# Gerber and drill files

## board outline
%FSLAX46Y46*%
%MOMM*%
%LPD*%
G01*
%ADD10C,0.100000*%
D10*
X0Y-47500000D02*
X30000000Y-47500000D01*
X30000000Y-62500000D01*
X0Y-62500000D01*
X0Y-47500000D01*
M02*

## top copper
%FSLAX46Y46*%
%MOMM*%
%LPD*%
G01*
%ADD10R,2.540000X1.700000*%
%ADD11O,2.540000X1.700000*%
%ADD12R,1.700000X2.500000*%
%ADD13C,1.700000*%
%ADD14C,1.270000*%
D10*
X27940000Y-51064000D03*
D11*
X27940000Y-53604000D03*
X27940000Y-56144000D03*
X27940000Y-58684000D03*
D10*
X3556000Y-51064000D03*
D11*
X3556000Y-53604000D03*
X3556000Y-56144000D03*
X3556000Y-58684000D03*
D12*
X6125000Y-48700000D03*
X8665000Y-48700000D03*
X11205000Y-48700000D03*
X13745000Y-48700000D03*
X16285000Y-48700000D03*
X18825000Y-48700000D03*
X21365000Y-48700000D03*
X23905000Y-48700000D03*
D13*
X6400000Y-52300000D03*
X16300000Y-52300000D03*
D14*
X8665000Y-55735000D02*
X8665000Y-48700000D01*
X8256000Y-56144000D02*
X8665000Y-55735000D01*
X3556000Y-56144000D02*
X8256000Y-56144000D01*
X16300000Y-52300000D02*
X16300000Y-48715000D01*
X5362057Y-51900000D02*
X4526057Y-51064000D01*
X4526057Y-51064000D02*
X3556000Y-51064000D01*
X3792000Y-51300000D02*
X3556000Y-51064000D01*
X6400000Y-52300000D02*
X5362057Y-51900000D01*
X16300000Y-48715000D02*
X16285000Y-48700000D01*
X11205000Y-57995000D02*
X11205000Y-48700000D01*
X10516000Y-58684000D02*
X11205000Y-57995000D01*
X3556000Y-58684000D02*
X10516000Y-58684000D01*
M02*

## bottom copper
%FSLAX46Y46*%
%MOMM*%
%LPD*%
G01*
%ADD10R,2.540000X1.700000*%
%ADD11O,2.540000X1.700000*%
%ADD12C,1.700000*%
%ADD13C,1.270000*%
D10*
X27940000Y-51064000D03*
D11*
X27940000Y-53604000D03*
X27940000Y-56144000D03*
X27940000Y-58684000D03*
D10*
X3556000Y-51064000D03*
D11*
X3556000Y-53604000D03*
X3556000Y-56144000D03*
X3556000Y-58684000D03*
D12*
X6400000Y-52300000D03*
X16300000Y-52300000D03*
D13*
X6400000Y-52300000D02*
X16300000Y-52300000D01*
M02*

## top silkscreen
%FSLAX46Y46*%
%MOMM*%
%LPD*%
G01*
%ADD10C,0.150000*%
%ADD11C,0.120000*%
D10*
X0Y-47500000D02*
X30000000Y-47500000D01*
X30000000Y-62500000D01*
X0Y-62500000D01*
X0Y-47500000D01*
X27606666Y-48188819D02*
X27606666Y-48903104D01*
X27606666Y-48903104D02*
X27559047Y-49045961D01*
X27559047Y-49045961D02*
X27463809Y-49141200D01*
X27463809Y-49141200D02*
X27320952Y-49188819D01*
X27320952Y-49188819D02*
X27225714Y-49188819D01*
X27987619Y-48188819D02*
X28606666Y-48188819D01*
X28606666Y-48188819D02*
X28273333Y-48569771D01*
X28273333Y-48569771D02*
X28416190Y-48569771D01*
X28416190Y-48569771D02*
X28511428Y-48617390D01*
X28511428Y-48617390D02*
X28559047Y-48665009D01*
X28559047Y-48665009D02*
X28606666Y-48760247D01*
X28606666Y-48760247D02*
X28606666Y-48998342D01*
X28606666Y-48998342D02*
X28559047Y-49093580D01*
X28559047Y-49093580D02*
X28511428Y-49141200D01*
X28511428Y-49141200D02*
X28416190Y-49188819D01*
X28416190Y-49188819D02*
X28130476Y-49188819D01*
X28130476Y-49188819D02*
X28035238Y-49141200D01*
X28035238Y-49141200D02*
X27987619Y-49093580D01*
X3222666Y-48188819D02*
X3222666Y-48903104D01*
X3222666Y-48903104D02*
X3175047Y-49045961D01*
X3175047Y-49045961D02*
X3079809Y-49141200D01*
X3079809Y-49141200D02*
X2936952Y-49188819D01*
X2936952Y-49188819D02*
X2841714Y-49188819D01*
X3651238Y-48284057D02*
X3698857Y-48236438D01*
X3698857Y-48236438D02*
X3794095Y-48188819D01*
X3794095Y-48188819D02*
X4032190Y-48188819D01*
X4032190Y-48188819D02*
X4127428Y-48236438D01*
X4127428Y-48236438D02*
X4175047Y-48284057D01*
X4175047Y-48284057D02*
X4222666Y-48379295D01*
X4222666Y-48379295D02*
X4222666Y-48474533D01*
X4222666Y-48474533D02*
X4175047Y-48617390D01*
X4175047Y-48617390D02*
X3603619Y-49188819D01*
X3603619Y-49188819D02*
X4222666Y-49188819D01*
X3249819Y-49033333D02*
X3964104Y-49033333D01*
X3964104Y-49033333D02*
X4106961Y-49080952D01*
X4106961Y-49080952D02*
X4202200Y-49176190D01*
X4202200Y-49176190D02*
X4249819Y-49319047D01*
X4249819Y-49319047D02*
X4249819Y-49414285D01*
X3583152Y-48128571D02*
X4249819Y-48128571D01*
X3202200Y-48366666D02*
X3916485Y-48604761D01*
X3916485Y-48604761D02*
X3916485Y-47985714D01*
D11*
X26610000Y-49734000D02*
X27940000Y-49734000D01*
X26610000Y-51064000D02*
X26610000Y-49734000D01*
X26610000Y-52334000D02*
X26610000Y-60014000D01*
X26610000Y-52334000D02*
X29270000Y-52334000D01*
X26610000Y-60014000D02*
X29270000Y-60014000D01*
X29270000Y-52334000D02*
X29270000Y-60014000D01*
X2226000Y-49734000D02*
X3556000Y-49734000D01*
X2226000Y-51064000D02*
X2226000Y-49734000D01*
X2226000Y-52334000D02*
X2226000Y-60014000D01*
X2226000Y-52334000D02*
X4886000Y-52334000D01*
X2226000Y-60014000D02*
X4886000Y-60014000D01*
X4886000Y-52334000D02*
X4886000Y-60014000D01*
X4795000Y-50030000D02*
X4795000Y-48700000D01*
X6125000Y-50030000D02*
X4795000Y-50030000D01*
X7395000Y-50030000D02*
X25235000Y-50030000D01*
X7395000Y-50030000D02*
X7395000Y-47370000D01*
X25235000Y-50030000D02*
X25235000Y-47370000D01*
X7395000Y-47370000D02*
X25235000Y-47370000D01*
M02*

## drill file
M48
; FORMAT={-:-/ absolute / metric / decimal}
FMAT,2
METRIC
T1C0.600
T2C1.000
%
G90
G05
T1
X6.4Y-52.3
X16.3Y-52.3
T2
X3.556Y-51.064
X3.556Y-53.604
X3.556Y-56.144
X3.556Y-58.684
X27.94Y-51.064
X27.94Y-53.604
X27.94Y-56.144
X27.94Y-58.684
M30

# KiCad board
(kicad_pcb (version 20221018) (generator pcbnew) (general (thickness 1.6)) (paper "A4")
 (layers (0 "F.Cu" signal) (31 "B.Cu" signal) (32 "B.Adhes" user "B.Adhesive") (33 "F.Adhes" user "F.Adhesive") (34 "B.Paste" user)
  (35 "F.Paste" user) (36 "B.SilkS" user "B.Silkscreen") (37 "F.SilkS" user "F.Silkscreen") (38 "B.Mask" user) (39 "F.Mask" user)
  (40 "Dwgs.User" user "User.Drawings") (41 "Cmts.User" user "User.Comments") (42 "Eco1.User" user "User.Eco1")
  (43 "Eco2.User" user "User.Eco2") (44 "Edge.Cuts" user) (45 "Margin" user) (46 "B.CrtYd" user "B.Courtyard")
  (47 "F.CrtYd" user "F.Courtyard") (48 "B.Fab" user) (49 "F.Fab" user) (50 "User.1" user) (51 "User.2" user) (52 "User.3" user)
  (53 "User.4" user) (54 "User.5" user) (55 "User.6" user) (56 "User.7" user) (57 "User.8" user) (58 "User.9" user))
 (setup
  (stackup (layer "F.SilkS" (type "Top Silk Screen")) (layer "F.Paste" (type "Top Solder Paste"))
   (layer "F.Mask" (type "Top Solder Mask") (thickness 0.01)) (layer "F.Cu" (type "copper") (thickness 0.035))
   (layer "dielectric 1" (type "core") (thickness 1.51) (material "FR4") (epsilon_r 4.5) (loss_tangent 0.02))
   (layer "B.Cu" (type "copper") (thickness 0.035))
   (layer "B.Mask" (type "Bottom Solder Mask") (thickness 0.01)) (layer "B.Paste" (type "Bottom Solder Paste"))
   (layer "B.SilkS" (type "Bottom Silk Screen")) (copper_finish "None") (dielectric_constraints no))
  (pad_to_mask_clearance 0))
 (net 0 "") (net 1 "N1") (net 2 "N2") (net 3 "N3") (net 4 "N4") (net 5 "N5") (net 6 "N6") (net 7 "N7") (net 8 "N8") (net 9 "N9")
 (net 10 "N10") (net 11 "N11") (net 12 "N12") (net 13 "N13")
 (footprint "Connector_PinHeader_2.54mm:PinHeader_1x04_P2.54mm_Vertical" (layer "F.Cu") (at 27.94 51.064)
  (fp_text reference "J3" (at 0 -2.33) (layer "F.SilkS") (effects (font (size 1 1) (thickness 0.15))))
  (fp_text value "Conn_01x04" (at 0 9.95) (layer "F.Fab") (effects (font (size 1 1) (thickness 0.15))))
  (fp_line (start -1.33 -1.33) (end 0 -1.33) (stroke (width 0.12) (type solid)) (layer "F.SilkS"))
  (fp_line (start -1.33 0) (end -1.33 -1.33) (stroke (width 0.12) (type solid)) (layer "F.SilkS"))
  (fp_line (start -1.33 1.27) (end -1.33 8.95) (stroke (width 0.12) (type solid)) (layer "F.SilkS"))
  (fp_line (start -1.33 1.27) (end 1.33 1.27) (stroke (width 0.12) (type solid)) (layer "F.SilkS"))
  (fp_line (start -1.33 8.95) (end 1.33 8.95) (stroke (width 0.12) (type solid)) (layer "F.SilkS"))
  (fp_line (start 1.33 1.27) (end 1.33 8.95) (stroke (width 0.12) (type solid)) (layer "F.SilkS"))
  (pad "1" thru_hole rect (at 0 0) (size 2.54 1.7) (drill 1) (layers "*.Cu" "*.Mask") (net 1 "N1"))
  (pad "2" thru_hole oval (at 0 2.54) (size 2.54 1.7) (drill 1) (layers "*.Cu" "*.Mask") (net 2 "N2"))
  (pad "3" thru_hole oval (at 0 5.08) (size 2.54 1.7) (drill 1) (layers "*.Cu" "*.Mask") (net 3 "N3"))
  (pad "4" thru_hole oval (at 0 7.62) (size 2.54 1.7) (drill 1) (layers "*.Cu" "*.Mask") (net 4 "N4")))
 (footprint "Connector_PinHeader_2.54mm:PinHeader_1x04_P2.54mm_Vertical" (layer "F.Cu") (at 3.556 51.064)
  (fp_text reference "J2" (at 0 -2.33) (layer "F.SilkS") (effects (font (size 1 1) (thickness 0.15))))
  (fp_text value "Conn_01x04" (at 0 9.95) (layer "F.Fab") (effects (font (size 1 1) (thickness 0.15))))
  (fp_line (start -1.33 -1.33) (end 0 -1.33) (stroke (width 0.12) (type solid)) (layer "F.SilkS"))
  (fp_line (start -1.33 0) (end -1.33 -1.33) (stroke (width 0.12) (type solid)) (layer "F.SilkS"))
  (fp_line (start -1.33 1.27) (end -1.33 8.95) (stroke (width 0.12) (type solid)) (layer "F.SilkS"))
  (fp_line (start -1.33 1.27) (end 1.33 1.27) (stroke (width 0.12) (type solid)) (layer "F.SilkS"))
  (fp_line (start -1.33 8.95) (end 1.33 8.95) (stroke (width 0.12) (type solid)) (layer "F.SilkS"))
  (fp_line (start 1.33 1.27) (end 1.33 8.95) (stroke (width 0.12) (type solid)) (layer "F.SilkS"))
  (pad "1" thru_hole rect (at 0 0) (size 2.54 1.7) (drill 1) (layers "*.Cu" "*.Mask") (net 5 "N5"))
  (pad "2" thru_hole oval (at 0 2.54) (size 2.54 1.7) (drill 1) (layers "*.Cu" "*.Mask") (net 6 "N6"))
  (pad "3" thru_hole oval (at 0 5.08) (size 2.54 1.7) (drill 1) (layers "*.Cu" "*.Mask") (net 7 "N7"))
  (pad "4" thru_hole oval (at 0 7.62) (size 2.54 1.7) (drill 1) (layers "*.Cu" "*.Mask") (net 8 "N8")))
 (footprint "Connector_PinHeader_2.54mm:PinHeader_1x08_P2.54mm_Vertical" (layer "F.Cu") (at 6.125 48.7 90)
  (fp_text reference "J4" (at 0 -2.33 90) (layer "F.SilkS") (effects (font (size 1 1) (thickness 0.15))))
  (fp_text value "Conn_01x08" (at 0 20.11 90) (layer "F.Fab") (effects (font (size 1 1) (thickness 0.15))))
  (fp_line (start -1.33 -1.33) (end 0 -1.33) (stroke (width 0.12) (type solid)) (layer "F.SilkS"))
  (fp_line (start -1.33 0) (end -1.33 -1.33) (stroke (width 0.12) (type solid)) (layer "F.SilkS"))
  (fp_line (start -1.33 1.27) (end -1.33 19.11) (stroke (width 0.12) (type solid)) (layer "F.SilkS"))
  (fp_line (start -1.33 1.27) (end 1.33 1.27) (stroke (width 0.12) (type solid)) (layer "F.SilkS"))
  (fp_line (start -1.33 19.11) (end 1.33 19.11) (stroke (width 0.12) (type solid)) (layer "F.SilkS"))
  (fp_line (start 1.33 1.27) (end 1.33 19.11) (stroke (width 0.12) (type solid)) (layer "F.SilkS"))
  (pad "1" smd rect (at 0 0 90) (size 2.5 1.7) (layers "F.Cu" "F.Paste" "F.Mask") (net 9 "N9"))
  (pad "2" smd rect (at 0 2.54 90) (size 2.5 1.7) (layers "F.Cu" "F.Paste" "F.Mask") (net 7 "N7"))
  (pad "3" smd rect (at 0 5.08 90) (size 2.5 1.7) (layers "F.Cu" "F.Paste" "F.Mask") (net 8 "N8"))
  (pad "4" smd rect (at 0 7.62 90) (size 2.5 1.7) (layers "F.Cu" "F.Paste" "F.Mask") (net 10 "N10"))
  (pad "5" smd rect (at 0 10.16 90) (size 2.5 1.7) (layers "F.Cu" "F.Paste" "F.Mask") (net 5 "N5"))
  (pad "6" smd rect (at 0 12.7 90) (size 2.5 1.7) (layers "F.Cu" "F.Paste" "F.Mask") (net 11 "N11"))
  (pad "7" smd rect (at 0 15.24 90) (size 2.5 1.7) (layers "F.Cu" "F.Paste" "F.Mask") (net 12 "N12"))
  (pad "8" smd rect (at 0 17.78 90) (size 2.5 1.7) (layers "F.Cu" "F.Paste" "F.Mask") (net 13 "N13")))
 (gr_rect (start 0 47.5) (end 30 62.5) (stroke (width 0.15) (type solid)) (fill none) (layer "F.SilkS"))
 (gr_rect (start 0 47.5) (end 30 62.5) (stroke (width 0.1) (type solid)) (fill none) (layer "Edge.Cuts"))
 (segment (start 8.665 55.735) (end 8.665 48.7) (width 1.27) (layer "F.Cu") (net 7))
 (segment (start 8.256 56.144) (end 8.665 55.735) (width 1.27) (layer "F.Cu") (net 7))
 (segment (start 3.556 56.144) (end 8.256 56.144) (width 1.27) (layer "F.Cu") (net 7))
 (segment (start 16.3 52.3) (end 16.3 48.715) (width 1.27) (layer "F.Cu") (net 5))
 (segment (start 5.362057 51.9) (end 4.526057 51.064) (width 1.27) (layer "F.Cu") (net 5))
 (segment (start 4.526057 51.064) (end 3.556 51.064) (width 1.27) (layer "F.Cu") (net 5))
 (segment (start 3.792 51.3) (end 3.556 51.064) (width 1.27) (layer "F.Cu") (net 5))
 (segment (start 6.4 52.3) (end 5.362057 51.9) (width 1.27) (layer "F.Cu") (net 5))
 (segment (start 16.3 48.715) (end 16.285 48.7) (width 1.27) (layer "F.Cu") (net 5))
 (via (at 6.4 52.3) (size 1.7) (drill 0.6) (layers "F.Cu" "B.Cu") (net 5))
 (via (at 16.3 52.3) (size 1.7) (drill 0.6) (layers "F.Cu" "B.Cu") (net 5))
 (segment (start 6.4 52.3) (end 16.3 52.3) (width 1.27) (layer "B.Cu") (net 5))
 (segment (start 11.205 57.995) (end 11.205 48.7) (width 1.27) (layer "F.Cu") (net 8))
 (segment (start 10.516 58.684) (end 11.205 57.995) (width 1.27) (layer "F.Cu") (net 8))
 (segment (start 3.556 58.684) (end 10.516 58.684) (width 1.27) (layer "F.Cu") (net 8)))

